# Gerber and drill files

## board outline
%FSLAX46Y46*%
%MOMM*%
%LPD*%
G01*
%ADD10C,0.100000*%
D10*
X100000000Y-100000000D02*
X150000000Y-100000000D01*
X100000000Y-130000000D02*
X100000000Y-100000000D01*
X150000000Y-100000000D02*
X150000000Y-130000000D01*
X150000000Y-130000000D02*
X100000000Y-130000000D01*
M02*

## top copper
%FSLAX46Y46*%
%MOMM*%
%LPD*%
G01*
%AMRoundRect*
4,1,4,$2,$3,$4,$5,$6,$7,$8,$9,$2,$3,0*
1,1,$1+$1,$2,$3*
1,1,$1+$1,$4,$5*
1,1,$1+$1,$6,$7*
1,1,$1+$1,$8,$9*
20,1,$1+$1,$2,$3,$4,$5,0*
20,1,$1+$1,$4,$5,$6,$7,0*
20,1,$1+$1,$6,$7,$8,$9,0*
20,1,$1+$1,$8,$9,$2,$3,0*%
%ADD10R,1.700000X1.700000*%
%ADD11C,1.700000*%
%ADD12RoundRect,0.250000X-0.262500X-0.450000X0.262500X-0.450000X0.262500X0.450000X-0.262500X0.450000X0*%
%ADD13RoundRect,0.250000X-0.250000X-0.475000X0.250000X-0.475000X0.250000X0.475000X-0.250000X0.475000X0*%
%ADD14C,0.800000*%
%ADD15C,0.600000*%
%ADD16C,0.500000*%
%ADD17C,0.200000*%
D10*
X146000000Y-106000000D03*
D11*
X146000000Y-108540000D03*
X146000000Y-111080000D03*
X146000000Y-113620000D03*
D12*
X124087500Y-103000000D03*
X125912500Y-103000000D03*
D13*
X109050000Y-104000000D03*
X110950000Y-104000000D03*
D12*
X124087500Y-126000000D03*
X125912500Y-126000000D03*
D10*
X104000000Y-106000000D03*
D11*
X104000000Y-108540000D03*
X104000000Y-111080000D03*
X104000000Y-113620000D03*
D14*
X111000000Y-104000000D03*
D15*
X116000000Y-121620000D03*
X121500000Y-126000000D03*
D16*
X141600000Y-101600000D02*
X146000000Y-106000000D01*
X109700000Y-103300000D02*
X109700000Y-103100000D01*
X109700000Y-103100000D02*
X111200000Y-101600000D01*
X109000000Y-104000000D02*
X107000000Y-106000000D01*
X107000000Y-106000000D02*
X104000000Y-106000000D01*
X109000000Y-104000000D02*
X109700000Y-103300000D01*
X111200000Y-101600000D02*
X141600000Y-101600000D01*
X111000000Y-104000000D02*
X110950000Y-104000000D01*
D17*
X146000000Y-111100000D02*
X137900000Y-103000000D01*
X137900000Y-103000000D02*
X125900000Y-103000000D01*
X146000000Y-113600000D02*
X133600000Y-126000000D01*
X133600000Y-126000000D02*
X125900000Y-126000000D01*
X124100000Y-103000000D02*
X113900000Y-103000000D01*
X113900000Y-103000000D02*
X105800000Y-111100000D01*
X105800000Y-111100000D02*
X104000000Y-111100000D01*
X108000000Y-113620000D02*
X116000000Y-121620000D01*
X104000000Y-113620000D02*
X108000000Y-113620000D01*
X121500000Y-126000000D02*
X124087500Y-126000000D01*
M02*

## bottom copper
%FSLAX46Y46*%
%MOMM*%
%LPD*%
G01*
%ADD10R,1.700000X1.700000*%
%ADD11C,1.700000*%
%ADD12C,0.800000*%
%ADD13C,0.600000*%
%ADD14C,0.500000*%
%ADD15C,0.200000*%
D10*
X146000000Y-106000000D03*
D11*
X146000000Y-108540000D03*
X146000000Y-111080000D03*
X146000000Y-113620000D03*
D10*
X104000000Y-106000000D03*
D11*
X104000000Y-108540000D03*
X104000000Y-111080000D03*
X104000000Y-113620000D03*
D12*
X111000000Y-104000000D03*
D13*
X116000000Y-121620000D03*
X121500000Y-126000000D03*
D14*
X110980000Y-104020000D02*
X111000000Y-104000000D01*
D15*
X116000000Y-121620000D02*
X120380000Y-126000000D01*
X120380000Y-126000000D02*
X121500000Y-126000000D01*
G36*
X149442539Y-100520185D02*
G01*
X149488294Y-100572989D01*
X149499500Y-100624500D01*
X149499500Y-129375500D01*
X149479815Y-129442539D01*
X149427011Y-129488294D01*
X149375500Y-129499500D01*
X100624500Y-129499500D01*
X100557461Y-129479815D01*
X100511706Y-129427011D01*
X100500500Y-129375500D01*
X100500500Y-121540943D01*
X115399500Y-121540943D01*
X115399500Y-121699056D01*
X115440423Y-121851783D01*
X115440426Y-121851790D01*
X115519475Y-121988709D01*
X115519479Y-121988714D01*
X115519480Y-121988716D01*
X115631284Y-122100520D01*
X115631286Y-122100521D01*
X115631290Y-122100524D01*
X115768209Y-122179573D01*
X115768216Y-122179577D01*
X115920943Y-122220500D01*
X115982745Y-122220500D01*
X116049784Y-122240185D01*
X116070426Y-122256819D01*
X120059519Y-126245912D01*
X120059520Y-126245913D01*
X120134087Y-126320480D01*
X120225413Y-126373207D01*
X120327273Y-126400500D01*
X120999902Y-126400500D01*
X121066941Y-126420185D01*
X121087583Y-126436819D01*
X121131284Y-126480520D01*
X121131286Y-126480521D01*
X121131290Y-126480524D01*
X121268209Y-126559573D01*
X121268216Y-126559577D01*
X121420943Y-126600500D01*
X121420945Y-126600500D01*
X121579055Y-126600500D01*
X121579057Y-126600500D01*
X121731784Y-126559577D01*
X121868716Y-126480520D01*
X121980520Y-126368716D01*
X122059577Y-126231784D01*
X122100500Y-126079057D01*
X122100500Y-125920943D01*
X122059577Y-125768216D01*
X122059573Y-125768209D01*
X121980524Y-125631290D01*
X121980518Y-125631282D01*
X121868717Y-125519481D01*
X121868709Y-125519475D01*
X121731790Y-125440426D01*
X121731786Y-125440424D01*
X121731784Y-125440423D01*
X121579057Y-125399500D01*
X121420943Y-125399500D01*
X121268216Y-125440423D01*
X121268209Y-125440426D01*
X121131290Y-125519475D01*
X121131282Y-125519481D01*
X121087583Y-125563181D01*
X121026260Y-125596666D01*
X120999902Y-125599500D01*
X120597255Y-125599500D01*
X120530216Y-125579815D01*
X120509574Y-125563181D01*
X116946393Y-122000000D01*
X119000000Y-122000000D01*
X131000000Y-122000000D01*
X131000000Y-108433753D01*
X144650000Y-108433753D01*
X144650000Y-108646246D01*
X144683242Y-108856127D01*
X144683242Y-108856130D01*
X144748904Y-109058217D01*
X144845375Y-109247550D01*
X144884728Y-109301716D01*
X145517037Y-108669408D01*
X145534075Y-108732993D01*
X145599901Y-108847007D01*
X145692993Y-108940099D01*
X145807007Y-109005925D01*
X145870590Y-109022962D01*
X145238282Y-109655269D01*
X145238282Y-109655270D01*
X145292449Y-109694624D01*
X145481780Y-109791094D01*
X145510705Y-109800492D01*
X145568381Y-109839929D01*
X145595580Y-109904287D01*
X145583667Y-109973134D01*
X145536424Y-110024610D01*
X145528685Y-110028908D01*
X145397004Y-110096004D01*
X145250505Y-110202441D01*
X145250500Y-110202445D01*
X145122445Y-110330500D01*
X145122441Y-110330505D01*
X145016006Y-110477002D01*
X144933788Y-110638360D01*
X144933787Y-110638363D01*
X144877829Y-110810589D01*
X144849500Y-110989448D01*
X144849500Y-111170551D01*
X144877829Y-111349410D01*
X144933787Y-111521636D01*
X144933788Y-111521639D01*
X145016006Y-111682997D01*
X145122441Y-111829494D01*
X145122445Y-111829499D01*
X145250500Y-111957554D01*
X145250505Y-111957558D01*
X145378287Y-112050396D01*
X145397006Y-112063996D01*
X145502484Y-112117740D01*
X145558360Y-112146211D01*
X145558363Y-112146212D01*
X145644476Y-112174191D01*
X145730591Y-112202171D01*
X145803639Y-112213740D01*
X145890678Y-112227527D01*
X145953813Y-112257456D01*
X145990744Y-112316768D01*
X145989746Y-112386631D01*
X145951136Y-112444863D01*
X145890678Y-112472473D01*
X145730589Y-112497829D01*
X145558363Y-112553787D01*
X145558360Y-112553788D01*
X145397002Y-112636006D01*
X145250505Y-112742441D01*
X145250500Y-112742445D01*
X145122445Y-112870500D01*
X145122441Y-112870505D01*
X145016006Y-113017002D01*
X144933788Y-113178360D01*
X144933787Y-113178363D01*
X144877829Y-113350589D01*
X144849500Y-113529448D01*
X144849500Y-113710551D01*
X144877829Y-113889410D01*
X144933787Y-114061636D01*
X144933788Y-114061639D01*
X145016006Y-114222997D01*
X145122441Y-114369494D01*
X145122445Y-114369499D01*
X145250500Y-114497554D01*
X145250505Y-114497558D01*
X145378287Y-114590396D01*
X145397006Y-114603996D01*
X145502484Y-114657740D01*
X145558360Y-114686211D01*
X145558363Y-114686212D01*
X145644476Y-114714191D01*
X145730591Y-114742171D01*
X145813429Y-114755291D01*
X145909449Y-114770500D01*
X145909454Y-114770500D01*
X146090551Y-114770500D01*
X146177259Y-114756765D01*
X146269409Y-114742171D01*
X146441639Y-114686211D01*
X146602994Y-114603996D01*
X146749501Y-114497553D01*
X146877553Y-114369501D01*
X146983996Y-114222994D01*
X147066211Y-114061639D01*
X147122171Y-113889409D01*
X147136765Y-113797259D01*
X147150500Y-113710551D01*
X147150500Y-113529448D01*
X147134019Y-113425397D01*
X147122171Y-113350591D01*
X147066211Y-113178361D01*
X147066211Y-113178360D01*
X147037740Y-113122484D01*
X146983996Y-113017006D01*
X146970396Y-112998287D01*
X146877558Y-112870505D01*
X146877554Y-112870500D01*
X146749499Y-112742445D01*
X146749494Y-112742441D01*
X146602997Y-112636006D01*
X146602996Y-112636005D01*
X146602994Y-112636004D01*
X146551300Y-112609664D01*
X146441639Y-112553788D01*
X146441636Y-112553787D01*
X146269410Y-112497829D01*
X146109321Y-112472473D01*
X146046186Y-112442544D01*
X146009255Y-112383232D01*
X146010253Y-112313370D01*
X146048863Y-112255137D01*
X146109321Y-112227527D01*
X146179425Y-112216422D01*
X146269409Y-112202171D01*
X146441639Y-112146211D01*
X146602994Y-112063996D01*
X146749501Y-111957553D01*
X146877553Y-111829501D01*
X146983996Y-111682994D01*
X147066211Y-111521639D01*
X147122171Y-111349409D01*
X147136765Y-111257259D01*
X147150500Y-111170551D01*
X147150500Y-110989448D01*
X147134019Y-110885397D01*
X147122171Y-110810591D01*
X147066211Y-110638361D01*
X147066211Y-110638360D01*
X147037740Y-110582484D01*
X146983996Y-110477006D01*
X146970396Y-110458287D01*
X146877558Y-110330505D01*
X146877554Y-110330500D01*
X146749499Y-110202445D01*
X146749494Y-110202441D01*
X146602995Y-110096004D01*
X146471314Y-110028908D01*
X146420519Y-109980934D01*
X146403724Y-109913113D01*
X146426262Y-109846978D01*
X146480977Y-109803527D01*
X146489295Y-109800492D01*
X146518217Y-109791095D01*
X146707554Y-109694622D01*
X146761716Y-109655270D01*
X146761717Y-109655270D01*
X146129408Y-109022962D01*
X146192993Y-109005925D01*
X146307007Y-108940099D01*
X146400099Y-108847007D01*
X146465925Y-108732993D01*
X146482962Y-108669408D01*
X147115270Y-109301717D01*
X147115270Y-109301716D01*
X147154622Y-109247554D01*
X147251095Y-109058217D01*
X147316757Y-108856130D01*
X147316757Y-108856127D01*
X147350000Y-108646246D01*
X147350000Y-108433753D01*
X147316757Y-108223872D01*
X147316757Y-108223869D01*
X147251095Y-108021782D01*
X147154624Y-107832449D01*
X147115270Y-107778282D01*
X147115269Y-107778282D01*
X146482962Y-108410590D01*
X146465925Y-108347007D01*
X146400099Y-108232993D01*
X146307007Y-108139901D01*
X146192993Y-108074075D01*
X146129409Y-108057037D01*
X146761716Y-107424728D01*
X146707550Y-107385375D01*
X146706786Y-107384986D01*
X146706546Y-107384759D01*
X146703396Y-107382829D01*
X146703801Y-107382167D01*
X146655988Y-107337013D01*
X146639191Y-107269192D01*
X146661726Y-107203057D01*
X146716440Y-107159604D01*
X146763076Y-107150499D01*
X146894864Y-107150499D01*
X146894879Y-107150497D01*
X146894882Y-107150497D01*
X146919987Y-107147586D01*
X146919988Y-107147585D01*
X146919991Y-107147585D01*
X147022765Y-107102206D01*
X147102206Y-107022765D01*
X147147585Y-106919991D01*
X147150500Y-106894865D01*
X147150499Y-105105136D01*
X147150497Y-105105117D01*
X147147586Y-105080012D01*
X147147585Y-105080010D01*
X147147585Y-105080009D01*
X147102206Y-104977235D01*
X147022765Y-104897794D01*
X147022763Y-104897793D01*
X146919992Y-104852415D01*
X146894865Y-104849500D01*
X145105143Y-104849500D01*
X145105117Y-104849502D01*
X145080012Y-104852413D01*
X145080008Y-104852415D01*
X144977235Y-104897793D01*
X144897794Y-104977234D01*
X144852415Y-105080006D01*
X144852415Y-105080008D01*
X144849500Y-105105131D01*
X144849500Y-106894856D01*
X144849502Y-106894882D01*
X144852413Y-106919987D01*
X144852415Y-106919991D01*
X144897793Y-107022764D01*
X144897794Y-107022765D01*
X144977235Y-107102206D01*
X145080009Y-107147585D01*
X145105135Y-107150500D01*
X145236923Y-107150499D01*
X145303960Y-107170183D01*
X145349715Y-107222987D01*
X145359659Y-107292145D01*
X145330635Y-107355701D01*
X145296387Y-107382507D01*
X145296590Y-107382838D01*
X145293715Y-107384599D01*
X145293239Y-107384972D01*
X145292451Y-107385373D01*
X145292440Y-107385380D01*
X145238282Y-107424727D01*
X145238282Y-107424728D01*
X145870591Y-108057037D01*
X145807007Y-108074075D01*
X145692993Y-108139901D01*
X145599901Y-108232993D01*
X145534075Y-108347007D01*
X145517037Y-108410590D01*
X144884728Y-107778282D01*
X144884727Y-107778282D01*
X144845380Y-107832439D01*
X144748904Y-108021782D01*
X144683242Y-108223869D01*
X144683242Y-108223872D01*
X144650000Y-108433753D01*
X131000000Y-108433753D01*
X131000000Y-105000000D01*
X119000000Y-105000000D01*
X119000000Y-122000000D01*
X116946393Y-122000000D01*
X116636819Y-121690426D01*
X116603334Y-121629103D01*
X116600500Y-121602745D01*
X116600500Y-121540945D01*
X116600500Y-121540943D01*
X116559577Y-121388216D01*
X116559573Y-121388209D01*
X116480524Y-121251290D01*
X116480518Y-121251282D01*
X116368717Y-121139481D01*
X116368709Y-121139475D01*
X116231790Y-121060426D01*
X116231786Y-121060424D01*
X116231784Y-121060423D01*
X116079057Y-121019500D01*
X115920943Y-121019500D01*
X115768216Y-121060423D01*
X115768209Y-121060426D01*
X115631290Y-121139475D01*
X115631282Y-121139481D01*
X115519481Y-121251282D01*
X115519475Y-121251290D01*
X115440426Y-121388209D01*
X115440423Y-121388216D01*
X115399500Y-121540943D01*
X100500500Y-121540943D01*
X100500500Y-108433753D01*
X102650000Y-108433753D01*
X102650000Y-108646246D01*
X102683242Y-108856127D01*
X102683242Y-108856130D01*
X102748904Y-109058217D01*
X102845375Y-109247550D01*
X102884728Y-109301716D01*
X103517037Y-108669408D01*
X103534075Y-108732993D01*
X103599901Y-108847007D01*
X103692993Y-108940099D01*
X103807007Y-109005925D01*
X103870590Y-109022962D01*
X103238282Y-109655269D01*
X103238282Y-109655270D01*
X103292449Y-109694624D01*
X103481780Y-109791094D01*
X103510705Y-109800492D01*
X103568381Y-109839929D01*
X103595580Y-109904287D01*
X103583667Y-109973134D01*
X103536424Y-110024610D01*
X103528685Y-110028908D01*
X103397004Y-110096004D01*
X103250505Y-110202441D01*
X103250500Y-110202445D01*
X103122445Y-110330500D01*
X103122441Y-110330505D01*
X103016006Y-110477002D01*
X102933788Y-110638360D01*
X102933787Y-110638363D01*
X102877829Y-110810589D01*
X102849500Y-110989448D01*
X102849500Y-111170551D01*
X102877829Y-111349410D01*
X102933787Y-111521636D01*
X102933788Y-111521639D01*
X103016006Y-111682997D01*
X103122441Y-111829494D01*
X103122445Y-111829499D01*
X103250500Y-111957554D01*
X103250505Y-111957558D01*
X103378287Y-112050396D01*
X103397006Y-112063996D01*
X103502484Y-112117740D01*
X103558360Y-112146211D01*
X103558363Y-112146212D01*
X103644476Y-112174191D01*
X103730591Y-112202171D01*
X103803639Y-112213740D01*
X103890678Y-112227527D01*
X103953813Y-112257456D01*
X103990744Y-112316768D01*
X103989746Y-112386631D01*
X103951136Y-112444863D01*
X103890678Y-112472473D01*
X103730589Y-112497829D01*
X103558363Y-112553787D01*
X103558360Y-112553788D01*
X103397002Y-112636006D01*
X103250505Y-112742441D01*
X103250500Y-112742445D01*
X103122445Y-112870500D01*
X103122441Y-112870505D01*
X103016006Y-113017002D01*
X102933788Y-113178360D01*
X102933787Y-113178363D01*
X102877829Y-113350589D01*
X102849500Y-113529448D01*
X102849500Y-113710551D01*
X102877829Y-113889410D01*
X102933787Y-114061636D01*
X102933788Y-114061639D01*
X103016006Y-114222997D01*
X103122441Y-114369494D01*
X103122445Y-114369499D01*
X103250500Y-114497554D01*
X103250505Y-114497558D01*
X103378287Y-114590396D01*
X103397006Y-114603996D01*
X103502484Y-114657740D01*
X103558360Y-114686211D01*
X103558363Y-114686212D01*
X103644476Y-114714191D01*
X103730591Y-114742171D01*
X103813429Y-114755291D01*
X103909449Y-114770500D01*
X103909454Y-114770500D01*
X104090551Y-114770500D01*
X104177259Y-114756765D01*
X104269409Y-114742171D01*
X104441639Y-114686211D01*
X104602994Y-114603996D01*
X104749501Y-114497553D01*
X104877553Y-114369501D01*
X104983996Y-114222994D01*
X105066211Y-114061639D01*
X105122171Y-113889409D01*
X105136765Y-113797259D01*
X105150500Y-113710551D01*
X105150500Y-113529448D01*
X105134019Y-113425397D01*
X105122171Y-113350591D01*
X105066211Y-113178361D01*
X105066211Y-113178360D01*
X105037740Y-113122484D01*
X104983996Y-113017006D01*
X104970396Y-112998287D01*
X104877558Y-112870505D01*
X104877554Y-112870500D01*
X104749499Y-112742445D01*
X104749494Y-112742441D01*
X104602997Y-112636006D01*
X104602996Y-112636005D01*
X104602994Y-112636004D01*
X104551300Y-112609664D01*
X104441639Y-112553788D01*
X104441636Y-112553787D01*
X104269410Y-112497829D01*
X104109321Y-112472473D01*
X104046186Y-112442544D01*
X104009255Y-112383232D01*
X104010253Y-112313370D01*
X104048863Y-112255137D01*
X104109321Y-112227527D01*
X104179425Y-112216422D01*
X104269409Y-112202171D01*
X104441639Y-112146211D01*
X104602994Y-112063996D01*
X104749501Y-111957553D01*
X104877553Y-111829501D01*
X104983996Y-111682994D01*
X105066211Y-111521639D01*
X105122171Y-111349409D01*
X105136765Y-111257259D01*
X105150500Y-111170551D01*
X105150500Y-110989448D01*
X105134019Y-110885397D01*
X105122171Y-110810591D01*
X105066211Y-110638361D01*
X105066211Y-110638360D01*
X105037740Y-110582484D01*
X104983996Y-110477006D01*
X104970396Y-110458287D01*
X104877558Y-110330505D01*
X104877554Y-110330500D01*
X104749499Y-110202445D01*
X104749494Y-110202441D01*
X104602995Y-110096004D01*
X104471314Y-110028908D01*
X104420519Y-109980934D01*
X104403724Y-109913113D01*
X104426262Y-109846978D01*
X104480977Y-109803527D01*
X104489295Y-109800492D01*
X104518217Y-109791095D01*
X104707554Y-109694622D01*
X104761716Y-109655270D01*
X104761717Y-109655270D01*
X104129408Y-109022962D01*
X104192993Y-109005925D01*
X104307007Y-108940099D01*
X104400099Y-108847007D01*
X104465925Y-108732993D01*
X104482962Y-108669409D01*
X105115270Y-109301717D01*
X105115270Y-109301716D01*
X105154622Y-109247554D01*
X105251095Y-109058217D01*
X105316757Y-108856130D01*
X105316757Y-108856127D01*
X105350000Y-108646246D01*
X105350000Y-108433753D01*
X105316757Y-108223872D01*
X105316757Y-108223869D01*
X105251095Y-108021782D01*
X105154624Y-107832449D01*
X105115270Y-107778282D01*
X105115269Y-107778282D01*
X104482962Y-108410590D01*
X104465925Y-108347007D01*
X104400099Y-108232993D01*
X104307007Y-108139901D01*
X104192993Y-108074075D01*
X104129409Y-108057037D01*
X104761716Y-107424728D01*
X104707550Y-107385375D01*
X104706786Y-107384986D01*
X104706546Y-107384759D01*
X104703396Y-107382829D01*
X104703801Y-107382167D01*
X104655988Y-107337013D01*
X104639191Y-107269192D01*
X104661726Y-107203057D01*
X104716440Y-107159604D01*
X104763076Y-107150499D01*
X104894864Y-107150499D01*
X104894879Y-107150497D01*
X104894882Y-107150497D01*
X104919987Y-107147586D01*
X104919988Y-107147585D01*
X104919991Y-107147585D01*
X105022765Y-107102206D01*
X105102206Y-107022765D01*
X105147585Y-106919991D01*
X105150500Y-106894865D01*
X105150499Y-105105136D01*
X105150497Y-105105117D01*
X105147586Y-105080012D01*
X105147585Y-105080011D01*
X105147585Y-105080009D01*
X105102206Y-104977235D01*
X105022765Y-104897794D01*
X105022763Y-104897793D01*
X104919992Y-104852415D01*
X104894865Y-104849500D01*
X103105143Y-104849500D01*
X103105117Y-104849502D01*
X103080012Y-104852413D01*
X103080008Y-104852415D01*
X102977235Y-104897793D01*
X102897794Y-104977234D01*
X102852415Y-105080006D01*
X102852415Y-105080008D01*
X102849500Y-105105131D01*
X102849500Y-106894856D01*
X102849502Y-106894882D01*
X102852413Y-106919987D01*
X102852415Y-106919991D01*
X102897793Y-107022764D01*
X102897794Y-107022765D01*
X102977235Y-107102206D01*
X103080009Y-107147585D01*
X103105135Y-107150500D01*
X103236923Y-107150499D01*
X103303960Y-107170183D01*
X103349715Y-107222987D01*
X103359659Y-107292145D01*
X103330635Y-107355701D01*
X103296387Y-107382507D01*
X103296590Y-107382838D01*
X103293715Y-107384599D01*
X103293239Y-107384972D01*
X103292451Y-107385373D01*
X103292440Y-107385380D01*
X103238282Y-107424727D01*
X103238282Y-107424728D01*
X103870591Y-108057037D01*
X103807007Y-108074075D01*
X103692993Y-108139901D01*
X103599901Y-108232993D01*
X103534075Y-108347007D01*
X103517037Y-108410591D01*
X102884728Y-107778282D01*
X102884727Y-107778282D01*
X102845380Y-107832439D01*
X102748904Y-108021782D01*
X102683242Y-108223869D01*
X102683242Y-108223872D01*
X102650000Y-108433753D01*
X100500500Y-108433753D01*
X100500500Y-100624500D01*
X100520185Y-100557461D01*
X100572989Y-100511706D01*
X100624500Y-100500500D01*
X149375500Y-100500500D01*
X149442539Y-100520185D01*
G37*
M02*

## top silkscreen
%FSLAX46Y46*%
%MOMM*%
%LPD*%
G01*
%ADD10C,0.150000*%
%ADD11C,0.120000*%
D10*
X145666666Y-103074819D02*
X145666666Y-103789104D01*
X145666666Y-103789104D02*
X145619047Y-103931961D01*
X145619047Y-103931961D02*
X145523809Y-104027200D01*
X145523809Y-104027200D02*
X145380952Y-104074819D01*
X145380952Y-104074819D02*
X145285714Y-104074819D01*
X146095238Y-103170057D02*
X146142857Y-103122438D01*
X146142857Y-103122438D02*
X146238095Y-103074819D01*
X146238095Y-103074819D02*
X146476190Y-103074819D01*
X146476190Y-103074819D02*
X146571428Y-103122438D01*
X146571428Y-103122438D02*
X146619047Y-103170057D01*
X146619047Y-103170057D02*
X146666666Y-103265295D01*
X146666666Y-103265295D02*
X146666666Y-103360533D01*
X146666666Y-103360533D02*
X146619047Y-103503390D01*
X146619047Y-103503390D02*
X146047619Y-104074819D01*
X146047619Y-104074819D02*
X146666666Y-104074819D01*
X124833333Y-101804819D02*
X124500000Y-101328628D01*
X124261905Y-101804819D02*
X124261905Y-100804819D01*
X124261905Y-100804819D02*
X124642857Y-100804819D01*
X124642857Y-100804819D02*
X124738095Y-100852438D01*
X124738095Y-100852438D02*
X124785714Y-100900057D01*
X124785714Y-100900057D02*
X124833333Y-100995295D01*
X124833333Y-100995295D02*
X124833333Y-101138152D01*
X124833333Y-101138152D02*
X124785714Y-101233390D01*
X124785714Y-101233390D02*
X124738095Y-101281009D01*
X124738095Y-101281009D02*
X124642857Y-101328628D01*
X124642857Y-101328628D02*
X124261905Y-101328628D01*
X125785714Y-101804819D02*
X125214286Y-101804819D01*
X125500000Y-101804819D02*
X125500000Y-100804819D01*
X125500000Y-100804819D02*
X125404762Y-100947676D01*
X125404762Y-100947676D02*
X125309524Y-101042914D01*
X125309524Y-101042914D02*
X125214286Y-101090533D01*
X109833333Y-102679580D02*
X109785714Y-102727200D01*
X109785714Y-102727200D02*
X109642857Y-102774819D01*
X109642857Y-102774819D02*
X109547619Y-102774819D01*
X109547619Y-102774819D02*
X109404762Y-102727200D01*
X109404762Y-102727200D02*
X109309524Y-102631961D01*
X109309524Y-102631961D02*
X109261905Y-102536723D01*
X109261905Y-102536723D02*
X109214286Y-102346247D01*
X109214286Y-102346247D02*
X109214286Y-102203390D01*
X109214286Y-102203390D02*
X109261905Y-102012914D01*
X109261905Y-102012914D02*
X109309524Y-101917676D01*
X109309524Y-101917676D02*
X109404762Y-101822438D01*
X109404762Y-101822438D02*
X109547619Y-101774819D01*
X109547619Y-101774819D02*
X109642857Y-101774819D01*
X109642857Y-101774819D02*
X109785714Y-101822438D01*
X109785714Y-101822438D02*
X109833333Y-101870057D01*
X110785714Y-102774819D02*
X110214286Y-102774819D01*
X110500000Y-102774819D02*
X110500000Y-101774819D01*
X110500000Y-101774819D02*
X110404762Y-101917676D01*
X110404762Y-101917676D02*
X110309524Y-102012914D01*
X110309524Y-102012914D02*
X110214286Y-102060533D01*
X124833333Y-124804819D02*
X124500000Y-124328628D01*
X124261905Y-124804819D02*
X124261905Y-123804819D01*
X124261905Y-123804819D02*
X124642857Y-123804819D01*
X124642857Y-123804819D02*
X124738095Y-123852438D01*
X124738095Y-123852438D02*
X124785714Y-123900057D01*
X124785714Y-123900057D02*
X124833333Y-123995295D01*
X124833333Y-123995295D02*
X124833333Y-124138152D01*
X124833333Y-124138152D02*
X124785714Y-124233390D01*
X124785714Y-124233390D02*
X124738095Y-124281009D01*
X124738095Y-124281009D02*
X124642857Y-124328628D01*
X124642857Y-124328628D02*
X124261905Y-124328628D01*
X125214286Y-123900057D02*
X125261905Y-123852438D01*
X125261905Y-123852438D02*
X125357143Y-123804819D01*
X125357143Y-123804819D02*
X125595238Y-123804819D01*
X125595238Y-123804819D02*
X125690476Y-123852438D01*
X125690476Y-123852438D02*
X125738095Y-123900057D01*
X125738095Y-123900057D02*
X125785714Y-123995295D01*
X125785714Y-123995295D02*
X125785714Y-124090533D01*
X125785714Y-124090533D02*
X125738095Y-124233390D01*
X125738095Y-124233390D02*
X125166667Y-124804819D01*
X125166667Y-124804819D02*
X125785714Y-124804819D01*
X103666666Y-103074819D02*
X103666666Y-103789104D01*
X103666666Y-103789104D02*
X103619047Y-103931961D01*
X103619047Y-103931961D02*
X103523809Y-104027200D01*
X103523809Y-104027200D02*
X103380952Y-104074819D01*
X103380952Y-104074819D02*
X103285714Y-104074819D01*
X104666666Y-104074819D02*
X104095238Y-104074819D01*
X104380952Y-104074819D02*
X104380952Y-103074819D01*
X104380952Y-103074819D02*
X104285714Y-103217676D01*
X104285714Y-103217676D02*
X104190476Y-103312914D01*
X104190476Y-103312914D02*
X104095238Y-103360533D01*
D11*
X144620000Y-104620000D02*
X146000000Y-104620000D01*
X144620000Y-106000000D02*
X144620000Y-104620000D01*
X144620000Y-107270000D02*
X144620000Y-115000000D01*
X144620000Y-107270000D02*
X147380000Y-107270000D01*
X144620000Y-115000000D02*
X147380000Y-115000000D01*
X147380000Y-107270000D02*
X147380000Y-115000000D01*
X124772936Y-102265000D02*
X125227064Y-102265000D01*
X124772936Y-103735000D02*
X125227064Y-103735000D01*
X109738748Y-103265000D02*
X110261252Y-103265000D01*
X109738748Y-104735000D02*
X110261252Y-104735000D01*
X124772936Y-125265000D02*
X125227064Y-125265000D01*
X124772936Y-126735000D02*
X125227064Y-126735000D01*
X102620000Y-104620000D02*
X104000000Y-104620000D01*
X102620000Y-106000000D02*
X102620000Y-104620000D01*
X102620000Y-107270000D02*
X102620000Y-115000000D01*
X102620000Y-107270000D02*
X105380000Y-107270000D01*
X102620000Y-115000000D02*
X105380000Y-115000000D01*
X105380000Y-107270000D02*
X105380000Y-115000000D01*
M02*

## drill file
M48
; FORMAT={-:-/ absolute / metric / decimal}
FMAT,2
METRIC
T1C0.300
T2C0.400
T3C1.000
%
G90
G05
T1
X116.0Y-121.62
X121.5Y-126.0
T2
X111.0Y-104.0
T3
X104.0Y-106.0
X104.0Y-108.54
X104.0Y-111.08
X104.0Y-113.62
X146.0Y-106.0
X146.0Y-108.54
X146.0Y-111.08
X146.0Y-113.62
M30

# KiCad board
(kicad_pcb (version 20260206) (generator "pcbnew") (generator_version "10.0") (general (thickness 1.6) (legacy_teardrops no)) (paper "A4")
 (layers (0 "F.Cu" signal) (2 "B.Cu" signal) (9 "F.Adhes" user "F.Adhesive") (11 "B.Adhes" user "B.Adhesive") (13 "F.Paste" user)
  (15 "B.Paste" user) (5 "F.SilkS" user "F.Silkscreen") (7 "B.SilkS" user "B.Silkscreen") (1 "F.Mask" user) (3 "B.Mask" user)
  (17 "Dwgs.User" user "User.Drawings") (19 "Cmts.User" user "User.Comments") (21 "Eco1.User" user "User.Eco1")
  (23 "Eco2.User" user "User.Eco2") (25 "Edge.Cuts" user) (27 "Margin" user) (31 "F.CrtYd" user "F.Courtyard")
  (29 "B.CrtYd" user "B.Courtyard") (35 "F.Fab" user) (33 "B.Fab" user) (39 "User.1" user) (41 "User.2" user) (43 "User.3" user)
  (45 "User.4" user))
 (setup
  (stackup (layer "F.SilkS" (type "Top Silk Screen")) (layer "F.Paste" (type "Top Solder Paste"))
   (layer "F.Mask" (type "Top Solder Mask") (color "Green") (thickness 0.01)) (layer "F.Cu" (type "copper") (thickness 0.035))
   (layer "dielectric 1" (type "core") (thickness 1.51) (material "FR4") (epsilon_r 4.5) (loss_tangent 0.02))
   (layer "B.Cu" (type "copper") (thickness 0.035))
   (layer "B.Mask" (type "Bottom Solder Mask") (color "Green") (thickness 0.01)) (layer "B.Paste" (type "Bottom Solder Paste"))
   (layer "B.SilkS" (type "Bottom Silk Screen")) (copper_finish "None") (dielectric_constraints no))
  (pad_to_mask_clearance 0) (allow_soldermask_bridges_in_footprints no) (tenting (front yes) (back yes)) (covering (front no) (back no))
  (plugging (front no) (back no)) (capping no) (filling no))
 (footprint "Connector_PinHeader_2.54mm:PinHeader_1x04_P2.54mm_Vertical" (layer "F.Cu") (at 146 106)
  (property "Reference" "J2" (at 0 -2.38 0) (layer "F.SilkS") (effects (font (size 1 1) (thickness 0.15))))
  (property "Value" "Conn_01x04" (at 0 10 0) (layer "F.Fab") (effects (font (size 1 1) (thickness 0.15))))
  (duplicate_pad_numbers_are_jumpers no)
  (fp_line (start -1.38 -1.38) (end 0 -1.38) (stroke (width 0.12) (type solid)) (layer "F.SilkS"))
  (fp_line (start -1.38 0) (end -1.38 -1.38) (stroke (width 0.12) (type solid)) (layer "F.SilkS"))
  (fp_line (start -1.38 1.27) (end -1.38 9) (stroke (width 0.12) (type solid)) (layer "F.SilkS"))
  (fp_line (start -1.38 1.27) (end 1.38 1.27) (stroke (width 0.12) (type solid)) (layer "F.SilkS"))
  (fp_line (start -1.38 9) (end 1.38 9) (stroke (width 0.12) (type solid)) (layer "F.SilkS"))
  (fp_line (start 1.38 1.27) (end 1.38 9) (stroke (width 0.12) (type solid)) (layer "F.SilkS"))
  (pad "1" thru_hole rect (at 0 0) (size 1.7 1.7) (drill 1) (layers "*.Cu" "*.Mask") (remove_unused_layers no) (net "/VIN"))
  (pad "2" thru_hole circle (at 0 2.54) (size 1.7 1.7) (drill 1) (layers "*.Cu" "*.Mask") (remove_unused_layers no) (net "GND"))
  (pad "3" thru_hole circle (at 0 5.08) (size 1.7 1.7) (drill 1) (layers "*.Cu" "*.Mask") (remove_unused_layers no) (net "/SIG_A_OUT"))
  (pad "4" thru_hole circle (at 0 7.62) (size 1.7 1.7) (drill 1) (layers "*.Cu" "*.Mask") (remove_unused_layers no) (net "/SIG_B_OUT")))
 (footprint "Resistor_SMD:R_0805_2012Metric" (layer "F.Cu") (at 125 103)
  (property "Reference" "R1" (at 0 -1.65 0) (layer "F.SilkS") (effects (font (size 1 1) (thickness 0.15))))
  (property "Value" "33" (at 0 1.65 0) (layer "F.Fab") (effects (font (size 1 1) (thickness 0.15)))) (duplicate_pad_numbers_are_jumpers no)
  (fp_line (start -0.227064 -0.735) (end 0.227064 -0.735) (stroke (width 0.12) (type solid)) (layer "F.SilkS"))
  (fp_line (start -0.227064 0.735) (end 0.227064 0.735) (stroke (width 0.12) (type solid)) (layer "F.SilkS"))
  (pad "1" smd roundrect (at -0.9125 0) (size 1.025 1.4) (layers "F.Cu" "F.Mask" "F.Paste") (roundrect_rratio 0.243902) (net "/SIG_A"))
  (pad "2" smd roundrect (at 0.9125 0) (size 1.025 1.4) (layers "F.Cu" "F.Mask" "F.Paste") (roundrect_rratio 0.243902) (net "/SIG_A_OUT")))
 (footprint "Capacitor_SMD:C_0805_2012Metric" (layer "F.Cu") (at 110 104)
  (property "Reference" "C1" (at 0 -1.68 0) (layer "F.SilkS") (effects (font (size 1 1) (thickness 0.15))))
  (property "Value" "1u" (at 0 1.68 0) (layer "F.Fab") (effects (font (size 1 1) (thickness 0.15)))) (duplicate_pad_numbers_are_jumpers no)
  (fp_line (start -0.261252 -0.735) (end 0.261252 -0.735) (stroke (width 0.12) (type solid)) (layer "F.SilkS"))
  (fp_line (start -0.261252 0.735) (end 0.261252 0.735) (stroke (width 0.12) (type solid)) (layer "F.SilkS"))
  (pad "1" smd roundrect (at -0.95 0) (size 1 1.45) (layers "F.Cu" "F.Mask" "F.Paste") (roundrect_rratio 0.25) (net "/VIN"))
  (pad "2" smd roundrect (at 0.95 0) (size 1 1.45) (layers "F.Cu" "F.Mask" "F.Paste") (roundrect_rratio 0.25) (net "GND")))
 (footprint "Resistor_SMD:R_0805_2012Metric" (layer "F.Cu") (at 125 126)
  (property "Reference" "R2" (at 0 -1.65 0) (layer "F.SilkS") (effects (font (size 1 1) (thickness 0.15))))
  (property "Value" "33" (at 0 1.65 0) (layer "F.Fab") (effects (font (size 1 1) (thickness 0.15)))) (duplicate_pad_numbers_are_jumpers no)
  (fp_line (start -0.227064 -0.735) (end 0.227064 -0.735) (stroke (width 0.12) (type solid)) (layer "F.SilkS"))
  (fp_line (start -0.227064 0.735) (end 0.227064 0.735) (stroke (width 0.12) (type solid)) (layer "F.SilkS"))
  (pad "1" smd roundrect (at -0.9125 0) (size 1.025 1.4) (layers "F.Cu" "F.Mask" "F.Paste") (roundrect_rratio 0.243902) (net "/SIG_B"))
  (pad "2" smd roundrect (at 0.9125 0) (size 1.025 1.4) (layers "F.Cu" "F.Mask" "F.Paste") (roundrect_rratio 0.243902) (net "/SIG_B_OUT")))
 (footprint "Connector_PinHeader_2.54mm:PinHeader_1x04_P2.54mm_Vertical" (layer "F.Cu") (at 104 106)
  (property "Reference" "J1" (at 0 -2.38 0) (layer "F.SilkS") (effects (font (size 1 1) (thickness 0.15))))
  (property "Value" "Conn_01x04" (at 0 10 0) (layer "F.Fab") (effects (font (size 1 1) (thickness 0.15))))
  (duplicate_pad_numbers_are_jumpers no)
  (fp_line (start -1.38 -1.38) (end 0 -1.38) (stroke (width 0.12) (type solid)) (layer "F.SilkS"))
  (fp_line (start -1.38 0) (end -1.38 -1.38) (stroke (width 0.12) (type solid)) (layer "F.SilkS"))
  (fp_line (start -1.38 1.27) (end -1.38 9) (stroke (width 0.12) (type solid)) (layer "F.SilkS"))
  (fp_line (start -1.38 1.27) (end 1.38 1.27) (stroke (width 0.12) (type solid)) (layer "F.SilkS"))
  (fp_line (start -1.38 9) (end 1.38 9) (stroke (width 0.12) (type solid)) (layer "F.SilkS"))
  (fp_line (start 1.38 1.27) (end 1.38 9) (stroke (width 0.12) (type solid)) (layer "F.SilkS"))
  (pad "1" thru_hole rect (at 0 0) (size 1.7 1.7) (drill 1) (layers "*.Cu" "*.Mask") (remove_unused_layers no) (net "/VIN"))
  (pad "2" thru_hole circle (at 0 2.54) (size 1.7 1.7) (drill 1) (layers "*.Cu" "*.Mask") (remove_unused_layers no) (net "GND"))
  (pad "3" thru_hole circle (at 0 5.08) (size 1.7 1.7) (drill 1) (layers "*.Cu" "*.Mask") (remove_unused_layers no) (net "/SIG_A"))
  (pad "4" thru_hole circle (at 0 7.62) (size 1.7 1.7) (drill 1) (layers "*.Cu" "*.Mask") (remove_unused_layers no) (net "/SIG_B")))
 (gr_line (start 100 100) (end 150 100) (stroke (width 0.1) (type default)) (layer "Edge.Cuts"))
 (gr_line (start 100 130) (end 100 100) (stroke (width 0.1) (type default)) (layer "Edge.Cuts"))
 (gr_line (start 150 100) (end 150 130) (stroke (width 0.1) (type default)) (layer "Edge.Cuts"))
 (gr_line (start 150 130) (end 100 130) (stroke (width 0.1) (type default)) (layer "Edge.Cuts"))
 (segment (start 141.6 101.6) (end 146 106) (width 0.5) (layer "F.Cu") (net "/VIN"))
 (segment (start 109.7 103.3) (end 109.7 103.1) (width 0.5) (layer "F.Cu") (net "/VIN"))
 (segment (start 109.7 103.1) (end 111.2 101.6) (width 0.5) (layer "F.Cu") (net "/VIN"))
 (segment (start 109 104) (end 107 106) (width 0.5) (layer "F.Cu") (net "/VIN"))
 (segment (start 107 106) (end 104 106) (width 0.5) (layer "F.Cu") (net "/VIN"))
 (segment (start 109 104) (end 109.7 103.3) (width 0.5) (layer "F.Cu") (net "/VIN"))
 (segment (start 111.2 101.6) (end 141.6 101.6) (width 0.5) (layer "F.Cu") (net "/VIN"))
 (segment (start 111 104) (end 110.95 104) (width 0.5) (layer "F.Cu") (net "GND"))
 (via (at 111 104) (size 0.8) (drill 0.4) (layers "F.Cu" "B.Cu") (capping yes) (filling yes) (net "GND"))
 (segment (start 110.98 104.02) (end 111 104) (width 0.5) (layer "B.Cu") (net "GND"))
 (segment (start 146 111.1) (end 137.9 103) (width 0.2) (layer "F.Cu") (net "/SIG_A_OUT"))
 (segment (start 137.9 103) (end 125.9 103) (width 0.2) (layer "F.Cu") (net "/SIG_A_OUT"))
 (segment (start 146 113.6) (end 133.6 126) (width 0.2) (layer "F.Cu") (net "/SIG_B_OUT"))
 (segment (start 133.6 126) (end 125.9 126) (width 0.2) (layer "F.Cu") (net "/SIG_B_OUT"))
 (segment (start 124.1 103) (end 113.9 103) (width 0.2) (layer "F.Cu") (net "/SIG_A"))
 (segment (start 113.9 103) (end 105.8 111.1) (width 0.2) (layer "F.Cu") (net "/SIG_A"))
 (segment (start 105.8 111.1) (end 104 111.1) (width 0.2) (layer "F.Cu") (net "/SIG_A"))
 (segment (start 108 113.62) (end 116 121.62) (width 0.2) (locked yes) (layer "F.Cu") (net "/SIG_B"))
 (segment (start 104 113.62) (end 108 113.62) (width 0.2) (locked yes) (layer "F.Cu") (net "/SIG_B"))
 (segment (start 121.5 126) (end 124.0875 126) (width 0.2) (locked yes) (layer "F.Cu") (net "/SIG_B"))
 (via (at 116 121.62) (size 0.6) (drill 0.3) (layers "F.Cu" "B.Cu") (locked yes) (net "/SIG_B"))
 (via (at 121.5 126) (size 0.6) (drill 0.3) (layers "F.Cu" "B.Cu") (locked yes) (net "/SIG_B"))
 (segment (start 116 121.62) (end 120.38 126) (width 0.2) (locked yes) (layer "B.Cu") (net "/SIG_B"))
 (segment (start 120.38 126) (end 121.5 126) (width 0.2) (locked yes) (layer "B.Cu") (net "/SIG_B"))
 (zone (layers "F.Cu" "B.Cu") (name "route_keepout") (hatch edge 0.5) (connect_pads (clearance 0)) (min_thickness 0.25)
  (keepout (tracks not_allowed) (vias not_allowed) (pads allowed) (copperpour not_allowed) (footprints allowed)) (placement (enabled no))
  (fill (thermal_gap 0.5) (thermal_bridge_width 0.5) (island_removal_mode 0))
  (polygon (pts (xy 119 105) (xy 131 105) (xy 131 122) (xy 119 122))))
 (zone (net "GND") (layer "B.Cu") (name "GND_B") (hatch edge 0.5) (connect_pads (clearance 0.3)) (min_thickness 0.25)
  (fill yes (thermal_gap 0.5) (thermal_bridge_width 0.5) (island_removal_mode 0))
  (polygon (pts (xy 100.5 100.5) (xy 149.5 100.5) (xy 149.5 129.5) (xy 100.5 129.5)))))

